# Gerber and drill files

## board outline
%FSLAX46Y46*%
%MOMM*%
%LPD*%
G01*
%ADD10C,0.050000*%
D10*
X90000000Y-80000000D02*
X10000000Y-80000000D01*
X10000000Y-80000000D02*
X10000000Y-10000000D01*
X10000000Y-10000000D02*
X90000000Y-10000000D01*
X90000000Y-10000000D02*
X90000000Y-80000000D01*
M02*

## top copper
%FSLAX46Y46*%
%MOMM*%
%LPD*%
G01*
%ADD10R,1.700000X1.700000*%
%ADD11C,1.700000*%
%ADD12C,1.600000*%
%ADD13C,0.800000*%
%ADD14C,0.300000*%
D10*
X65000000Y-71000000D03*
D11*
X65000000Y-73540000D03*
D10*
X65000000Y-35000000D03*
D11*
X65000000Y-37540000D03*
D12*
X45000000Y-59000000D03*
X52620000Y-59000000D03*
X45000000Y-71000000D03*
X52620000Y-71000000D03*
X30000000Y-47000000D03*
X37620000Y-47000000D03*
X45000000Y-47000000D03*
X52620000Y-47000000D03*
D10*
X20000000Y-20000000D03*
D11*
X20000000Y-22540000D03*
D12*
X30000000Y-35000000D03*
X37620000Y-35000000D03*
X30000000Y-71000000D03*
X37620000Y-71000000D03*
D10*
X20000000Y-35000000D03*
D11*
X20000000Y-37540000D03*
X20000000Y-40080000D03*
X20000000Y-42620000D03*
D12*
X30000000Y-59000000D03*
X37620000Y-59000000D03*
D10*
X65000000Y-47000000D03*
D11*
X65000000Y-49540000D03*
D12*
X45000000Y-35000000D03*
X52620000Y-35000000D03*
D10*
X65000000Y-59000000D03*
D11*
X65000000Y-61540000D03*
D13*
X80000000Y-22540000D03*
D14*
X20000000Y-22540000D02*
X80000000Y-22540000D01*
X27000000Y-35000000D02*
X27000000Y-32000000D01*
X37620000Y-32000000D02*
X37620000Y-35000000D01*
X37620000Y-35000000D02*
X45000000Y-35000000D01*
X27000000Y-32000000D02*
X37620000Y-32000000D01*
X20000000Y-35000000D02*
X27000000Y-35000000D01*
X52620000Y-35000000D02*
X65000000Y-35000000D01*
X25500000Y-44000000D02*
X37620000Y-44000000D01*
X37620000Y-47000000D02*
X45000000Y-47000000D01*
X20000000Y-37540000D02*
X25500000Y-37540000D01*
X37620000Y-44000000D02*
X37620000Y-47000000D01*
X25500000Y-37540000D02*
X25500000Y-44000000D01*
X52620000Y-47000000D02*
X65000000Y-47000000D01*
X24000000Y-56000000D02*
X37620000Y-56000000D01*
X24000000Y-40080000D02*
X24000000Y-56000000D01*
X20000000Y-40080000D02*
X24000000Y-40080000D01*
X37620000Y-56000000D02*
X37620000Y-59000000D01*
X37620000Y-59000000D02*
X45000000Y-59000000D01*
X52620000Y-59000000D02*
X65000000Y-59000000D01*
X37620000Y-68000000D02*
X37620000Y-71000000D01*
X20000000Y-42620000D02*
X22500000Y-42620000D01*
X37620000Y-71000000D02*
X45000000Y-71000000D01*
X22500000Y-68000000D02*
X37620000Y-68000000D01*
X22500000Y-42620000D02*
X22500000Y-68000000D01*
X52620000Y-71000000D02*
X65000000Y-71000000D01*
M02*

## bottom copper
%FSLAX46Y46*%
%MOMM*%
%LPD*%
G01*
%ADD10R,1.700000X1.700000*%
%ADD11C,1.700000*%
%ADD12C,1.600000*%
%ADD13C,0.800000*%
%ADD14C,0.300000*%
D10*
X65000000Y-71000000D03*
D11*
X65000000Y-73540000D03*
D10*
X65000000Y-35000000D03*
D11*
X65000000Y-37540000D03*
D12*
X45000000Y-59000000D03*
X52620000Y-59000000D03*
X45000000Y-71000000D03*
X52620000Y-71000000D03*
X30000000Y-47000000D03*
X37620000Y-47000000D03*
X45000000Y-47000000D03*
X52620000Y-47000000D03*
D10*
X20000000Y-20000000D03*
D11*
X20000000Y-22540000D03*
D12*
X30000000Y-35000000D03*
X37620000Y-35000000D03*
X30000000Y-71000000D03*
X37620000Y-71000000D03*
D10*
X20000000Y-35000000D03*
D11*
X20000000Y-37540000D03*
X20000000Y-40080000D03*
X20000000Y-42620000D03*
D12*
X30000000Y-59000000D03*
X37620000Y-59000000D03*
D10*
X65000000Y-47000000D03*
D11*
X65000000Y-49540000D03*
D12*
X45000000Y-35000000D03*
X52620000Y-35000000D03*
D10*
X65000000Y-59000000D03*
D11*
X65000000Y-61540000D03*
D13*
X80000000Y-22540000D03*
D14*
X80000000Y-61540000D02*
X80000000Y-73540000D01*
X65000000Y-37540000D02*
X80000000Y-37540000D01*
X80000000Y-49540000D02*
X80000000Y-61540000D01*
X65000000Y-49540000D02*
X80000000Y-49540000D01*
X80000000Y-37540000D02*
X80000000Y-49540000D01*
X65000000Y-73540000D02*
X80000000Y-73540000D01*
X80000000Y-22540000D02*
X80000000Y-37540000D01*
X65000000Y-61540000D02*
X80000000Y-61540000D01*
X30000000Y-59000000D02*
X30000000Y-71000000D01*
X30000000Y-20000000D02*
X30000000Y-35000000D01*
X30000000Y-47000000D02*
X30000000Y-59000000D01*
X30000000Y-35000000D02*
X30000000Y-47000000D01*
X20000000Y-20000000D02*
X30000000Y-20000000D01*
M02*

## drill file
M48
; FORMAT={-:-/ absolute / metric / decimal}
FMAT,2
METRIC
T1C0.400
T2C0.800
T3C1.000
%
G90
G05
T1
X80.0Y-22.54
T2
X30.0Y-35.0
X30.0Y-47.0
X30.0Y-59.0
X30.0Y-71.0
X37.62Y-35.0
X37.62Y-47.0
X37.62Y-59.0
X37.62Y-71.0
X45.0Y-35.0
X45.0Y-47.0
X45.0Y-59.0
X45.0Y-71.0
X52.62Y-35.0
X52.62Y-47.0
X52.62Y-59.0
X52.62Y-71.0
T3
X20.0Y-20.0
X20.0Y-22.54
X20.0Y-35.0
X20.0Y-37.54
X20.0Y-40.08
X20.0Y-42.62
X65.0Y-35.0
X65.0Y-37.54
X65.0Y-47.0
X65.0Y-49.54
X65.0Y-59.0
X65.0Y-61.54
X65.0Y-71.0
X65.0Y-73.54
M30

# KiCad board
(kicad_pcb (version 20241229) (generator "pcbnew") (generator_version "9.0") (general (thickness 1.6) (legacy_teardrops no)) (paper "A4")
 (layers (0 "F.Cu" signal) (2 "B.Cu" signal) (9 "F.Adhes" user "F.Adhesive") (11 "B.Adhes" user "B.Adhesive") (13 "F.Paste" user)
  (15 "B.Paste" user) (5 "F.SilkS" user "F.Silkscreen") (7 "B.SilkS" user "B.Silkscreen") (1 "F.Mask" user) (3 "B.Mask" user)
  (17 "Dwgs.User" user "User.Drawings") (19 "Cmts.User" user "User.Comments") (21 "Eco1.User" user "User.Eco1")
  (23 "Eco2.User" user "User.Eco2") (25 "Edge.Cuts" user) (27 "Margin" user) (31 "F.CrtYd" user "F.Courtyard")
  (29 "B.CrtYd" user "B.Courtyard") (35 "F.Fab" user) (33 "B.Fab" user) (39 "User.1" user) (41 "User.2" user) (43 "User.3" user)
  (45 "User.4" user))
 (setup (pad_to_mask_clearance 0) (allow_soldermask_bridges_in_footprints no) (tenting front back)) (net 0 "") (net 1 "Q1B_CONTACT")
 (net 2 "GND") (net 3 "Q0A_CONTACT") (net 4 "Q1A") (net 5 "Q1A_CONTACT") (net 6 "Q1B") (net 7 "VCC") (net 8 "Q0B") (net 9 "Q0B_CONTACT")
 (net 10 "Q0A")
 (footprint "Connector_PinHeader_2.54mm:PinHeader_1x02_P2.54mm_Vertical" (layer "F.Cu") (at 65 71)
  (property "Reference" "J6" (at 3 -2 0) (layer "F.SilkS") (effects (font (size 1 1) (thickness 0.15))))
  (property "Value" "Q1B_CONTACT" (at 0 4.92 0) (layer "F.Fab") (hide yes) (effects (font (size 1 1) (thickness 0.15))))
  (pad "1" thru_hole rect (at 0 0) (size 1.7 1.7) (drill 1) (layers "*.Cu" "*.Mask") (remove_unused_layers no) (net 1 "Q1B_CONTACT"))
  (pad "2" thru_hole circle (at 0 2.54) (size 1.7 1.7) (drill 1) (layers "*.Cu" "*.Mask") (remove_unused_layers no) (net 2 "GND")))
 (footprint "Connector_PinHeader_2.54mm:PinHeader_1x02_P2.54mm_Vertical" (layer "F.Cu") (at 65 35)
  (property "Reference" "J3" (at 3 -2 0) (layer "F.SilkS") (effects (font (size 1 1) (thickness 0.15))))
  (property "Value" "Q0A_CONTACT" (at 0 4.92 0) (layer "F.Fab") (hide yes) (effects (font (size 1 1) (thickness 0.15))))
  (pad "1" thru_hole rect (at 0 0) (size 1.7 1.7) (drill 1) (layers "*.Cu" "*.Mask") (remove_unused_layers no) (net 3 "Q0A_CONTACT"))
  (pad "2" thru_hole circle (at 0 2.54) (size 1.7 1.7) (drill 1) (layers "*.Cu" "*.Mask") (remove_unused_layers no) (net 2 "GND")))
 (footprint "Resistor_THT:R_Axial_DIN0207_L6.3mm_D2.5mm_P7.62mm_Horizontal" (layer "F.Cu") (at 45 59)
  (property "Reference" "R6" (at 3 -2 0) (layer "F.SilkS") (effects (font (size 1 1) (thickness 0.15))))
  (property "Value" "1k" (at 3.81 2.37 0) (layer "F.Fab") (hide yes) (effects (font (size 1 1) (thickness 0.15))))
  (pad "1" thru_hole circle (at 0 0) (size 1.6 1.6) (drill 0.8) (layers "*.Cu" "*.Mask") (remove_unused_layers no) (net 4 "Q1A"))
  (pad "2" thru_hole circle (at 7.62 0) (size 1.6 1.6) (drill 0.8) (layers "*.Cu" "*.Mask") (remove_unused_layers no) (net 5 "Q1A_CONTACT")))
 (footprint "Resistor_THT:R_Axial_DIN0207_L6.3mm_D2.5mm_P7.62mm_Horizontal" (layer "F.Cu") (at 45 71)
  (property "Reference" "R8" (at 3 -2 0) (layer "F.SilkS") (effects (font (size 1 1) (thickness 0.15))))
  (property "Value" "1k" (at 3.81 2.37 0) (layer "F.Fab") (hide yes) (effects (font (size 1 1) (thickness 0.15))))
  (pad "1" thru_hole circle (at 0 0) (size 1.6 1.6) (drill 0.8) (layers "*.Cu" "*.Mask") (remove_unused_layers no) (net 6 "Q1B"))
  (pad "2" thru_hole circle (at 7.62 0) (size 1.6 1.6) (drill 0.8) (layers "*.Cu" "*.Mask") (remove_unused_layers no) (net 1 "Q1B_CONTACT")))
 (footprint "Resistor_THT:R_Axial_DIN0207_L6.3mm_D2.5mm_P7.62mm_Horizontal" (layer "F.Cu") (at 30 47)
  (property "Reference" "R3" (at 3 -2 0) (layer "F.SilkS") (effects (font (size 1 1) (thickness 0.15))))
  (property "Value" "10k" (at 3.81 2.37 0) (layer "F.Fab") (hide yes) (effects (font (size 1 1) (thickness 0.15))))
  (pad "1" thru_hole circle (at 0 0) (size 1.6 1.6) (drill 0.8) (layers "*.Cu" "*.Mask") (remove_unused_layers no) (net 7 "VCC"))
  (pad "2" thru_hole circle (at 7.62 0) (size 1.6 1.6) (drill 0.8) (layers "*.Cu" "*.Mask") (remove_unused_layers no) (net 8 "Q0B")))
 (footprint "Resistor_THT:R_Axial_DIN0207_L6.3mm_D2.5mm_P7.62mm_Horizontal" (layer "F.Cu") (at 45 47)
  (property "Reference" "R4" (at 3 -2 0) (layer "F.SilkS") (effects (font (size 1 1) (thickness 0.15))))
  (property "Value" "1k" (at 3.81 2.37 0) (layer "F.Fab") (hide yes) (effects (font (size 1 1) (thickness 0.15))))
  (pad "1" thru_hole circle (at 0 0) (size 1.6 1.6) (drill 0.8) (layers "*.Cu" "*.Mask") (remove_unused_layers no) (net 8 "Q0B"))
  (pad "2" thru_hole circle (at 7.62 0) (size 1.6 1.6) (drill 0.8) (layers "*.Cu" "*.Mask") (remove_unused_layers no) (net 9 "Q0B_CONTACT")))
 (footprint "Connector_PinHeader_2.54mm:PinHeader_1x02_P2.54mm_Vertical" (layer "F.Cu") (at 20 20)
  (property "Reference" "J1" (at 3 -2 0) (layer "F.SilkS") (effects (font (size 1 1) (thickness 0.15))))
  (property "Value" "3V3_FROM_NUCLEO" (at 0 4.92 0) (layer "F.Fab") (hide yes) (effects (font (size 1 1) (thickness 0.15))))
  (pad "1" thru_hole rect (at 0 0) (size 1.7 1.7) (drill 1) (layers "*.Cu" "*.Mask") (remove_unused_layers no) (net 7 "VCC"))
  (pad "2" thru_hole circle (at 0 2.54) (size 1.7 1.7) (drill 1) (layers "*.Cu" "*.Mask") (remove_unused_layers no) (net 2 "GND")))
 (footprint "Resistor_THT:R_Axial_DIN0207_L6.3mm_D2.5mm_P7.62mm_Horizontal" (layer "F.Cu") (at 30 35)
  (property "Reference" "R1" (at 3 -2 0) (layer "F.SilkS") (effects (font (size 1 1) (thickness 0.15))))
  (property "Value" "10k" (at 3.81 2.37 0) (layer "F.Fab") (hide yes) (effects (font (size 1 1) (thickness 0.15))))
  (pad "1" thru_hole circle (at 0 0) (size 1.6 1.6) (drill 0.8) (layers "*.Cu" "*.Mask") (remove_unused_layers no) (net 7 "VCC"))
  (pad "2" thru_hole circle (at 7.62 0) (size 1.6 1.6) (drill 0.8) (layers "*.Cu" "*.Mask") (remove_unused_layers no) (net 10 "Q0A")))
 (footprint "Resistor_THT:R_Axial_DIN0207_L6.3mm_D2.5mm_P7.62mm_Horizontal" (layer "F.Cu") (at 30 71)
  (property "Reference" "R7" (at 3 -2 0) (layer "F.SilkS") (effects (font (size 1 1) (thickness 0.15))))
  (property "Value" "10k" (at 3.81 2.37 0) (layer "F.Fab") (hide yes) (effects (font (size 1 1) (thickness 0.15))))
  (pad "1" thru_hole circle (at 0 0) (size 1.6 1.6) (drill 0.8) (layers "*.Cu" "*.Mask") (remove_unused_layers no) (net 7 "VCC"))
  (pad "2" thru_hole circle (at 7.62 0) (size 1.6 1.6) (drill 0.8) (layers "*.Cu" "*.Mask") (remove_unused_layers no) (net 6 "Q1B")))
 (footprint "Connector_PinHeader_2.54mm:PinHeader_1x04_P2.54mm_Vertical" (layer "F.Cu") (at 20 35)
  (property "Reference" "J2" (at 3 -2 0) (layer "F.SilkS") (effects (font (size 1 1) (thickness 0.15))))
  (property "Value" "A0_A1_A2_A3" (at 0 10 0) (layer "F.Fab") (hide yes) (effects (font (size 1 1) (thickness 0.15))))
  (pad "1" thru_hole rect (at 0 0) (size 1.7 1.7) (drill 1) (layers "*.Cu" "*.Mask") (remove_unused_layers no) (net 10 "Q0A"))
  (pad "2" thru_hole circle (at 0 2.54) (size 1.7 1.7) (drill 1) (layers "*.Cu" "*.Mask") (remove_unused_layers no) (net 8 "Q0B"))
  (pad "3" thru_hole circle (at 0 5.08) (size 1.7 1.7) (drill 1) (layers "*.Cu" "*.Mask") (remove_unused_layers no) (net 4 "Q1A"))
  (pad "4" thru_hole circle (at 0 7.62) (size 1.7 1.7) (drill 1) (layers "*.Cu" "*.Mask") (remove_unused_layers no) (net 6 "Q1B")))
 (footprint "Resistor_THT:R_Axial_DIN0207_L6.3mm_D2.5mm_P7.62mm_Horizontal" (layer "F.Cu") (at 30 59)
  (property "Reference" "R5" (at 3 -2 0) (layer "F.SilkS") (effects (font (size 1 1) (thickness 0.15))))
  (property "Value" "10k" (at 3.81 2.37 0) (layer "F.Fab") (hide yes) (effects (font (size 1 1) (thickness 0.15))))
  (pad "1" thru_hole circle (at 0 0) (size 1.6 1.6) (drill 0.8) (layers "*.Cu" "*.Mask") (remove_unused_layers no) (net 7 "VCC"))
  (pad "2" thru_hole circle (at 7.62 0) (size 1.6 1.6) (drill 0.8) (layers "*.Cu" "*.Mask") (remove_unused_layers no) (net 4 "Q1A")))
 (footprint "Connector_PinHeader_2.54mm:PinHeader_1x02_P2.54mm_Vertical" (layer "F.Cu") (at 65 47)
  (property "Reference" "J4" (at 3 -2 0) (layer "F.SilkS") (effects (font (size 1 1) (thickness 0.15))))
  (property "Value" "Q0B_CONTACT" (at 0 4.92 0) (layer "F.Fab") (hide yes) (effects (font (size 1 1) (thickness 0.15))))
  (pad "1" thru_hole rect (at 0 0) (size 1.7 1.7) (drill 1) (layers "*.Cu" "*.Mask") (remove_unused_layers no) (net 9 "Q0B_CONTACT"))
  (pad "2" thru_hole circle (at 0 2.54) (size 1.7 1.7) (drill 1) (layers "*.Cu" "*.Mask") (remove_unused_layers no) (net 2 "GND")))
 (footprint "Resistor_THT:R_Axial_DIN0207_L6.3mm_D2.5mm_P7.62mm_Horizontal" (layer "F.Cu") (at 45 35)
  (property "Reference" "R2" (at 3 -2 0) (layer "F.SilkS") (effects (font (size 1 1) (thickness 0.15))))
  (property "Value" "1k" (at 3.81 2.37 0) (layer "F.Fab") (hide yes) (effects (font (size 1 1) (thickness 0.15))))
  (pad "1" thru_hole circle (at 0 0) (size 1.6 1.6) (drill 0.8) (layers "*.Cu" "*.Mask") (remove_unused_layers no) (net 10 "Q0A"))
  (pad "2" thru_hole circle (at 7.62 0) (size 1.6 1.6) (drill 0.8) (layers "*.Cu" "*.Mask") (remove_unused_layers no) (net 3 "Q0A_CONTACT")))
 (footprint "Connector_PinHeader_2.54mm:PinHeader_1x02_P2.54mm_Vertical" (layer "F.Cu") (at 65 59)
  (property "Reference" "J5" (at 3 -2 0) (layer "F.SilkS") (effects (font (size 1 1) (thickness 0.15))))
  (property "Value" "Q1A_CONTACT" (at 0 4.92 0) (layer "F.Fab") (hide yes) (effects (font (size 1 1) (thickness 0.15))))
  (pad "1" thru_hole rect (at 0 0) (size 1.7 1.7) (drill 1) (layers "*.Cu" "*.Mask") (remove_unused_layers no) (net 5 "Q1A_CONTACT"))
  (pad "2" thru_hole circle (at 0 2.54) (size 1.7 1.7) (drill 1) (layers "*.Cu" "*.Mask") (remove_unused_layers no) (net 2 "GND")))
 (gr_line (start 90 80) (end 10 80) (stroke (width 0.05) (type default)) (layer "Edge.Cuts"))
 (gr_line (start 10 80) (end 10 10) (stroke (width 0.05) (type default)) (layer "Edge.Cuts"))
 (gr_line (start 10 10) (end 90 10) (stroke (width 0.05) (type default)) (layer "Edge.Cuts"))
 (gr_line (start 90 10) (end 90 80) (stroke (width 0.05) (type default)) (layer "Edge.Cuts"))
 (segment (start 20 22.54) (end 80 22.54) (width 0.3) (layer "F.Cu") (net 2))
 (via (at 80 22.54) (size 0.8) (drill 0.4) (layers "F.Cu" "B.Cu") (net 2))
 (segment (start 80 61.54) (end 80 73.54) (width 0.3) (layer "B.Cu") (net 2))
 (segment (start 65 37.54) (end 80 37.54) (width 0.3) (layer "B.Cu") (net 2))
 (segment (start 80 49.54) (end 80 61.54) (width 0.3) (layer "B.Cu") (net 2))
 (segment (start 65 49.54) (end 80 49.54) (width 0.3) (layer "B.Cu") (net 2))
 (segment (start 80 37.54) (end 80 49.54) (width 0.3) (layer "B.Cu") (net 2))
 (segment (start 65 73.54) (end 80 73.54) (width 0.3) (layer "B.Cu") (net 2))
 (segment (start 80 22.54) (end 80 37.54) (width 0.3) (layer "B.Cu") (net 2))
 (segment (start 65 61.54) (end 80 61.54) (width 0.3) (layer "B.Cu") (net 2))
 (segment (start 27 35) (end 27 32) (width 0.3) (layer "F.Cu") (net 10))
 (segment (start 37.62 32) (end 37.62 35) (width 0.3) (layer "F.Cu") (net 10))
 (segment (start 37.62 35) (end 45 35) (width 0.3) (layer "F.Cu") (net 10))
 (segment (start 27 32) (end 37.62 32) (width 0.3) (layer "F.Cu") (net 10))
 (segment (start 20 35) (end 27 35) (width 0.3) (layer "F.Cu") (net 10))
 (segment (start 52.62 35) (end 65 35) (width 0.3) (layer "F.Cu") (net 3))
 (segment (start 25.5 44) (end 37.62 44) (width 0.3) (layer "F.Cu") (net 8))
 (segment (start 37.62 47) (end 45 47) (width 0.3) (layer "F.Cu") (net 8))
 (segment (start 20 37.54) (end 25.5 37.54) (width 0.3) (layer "F.Cu") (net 8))
 (segment (start 37.62 44) (end 37.62 47) (width 0.3) (layer "F.Cu") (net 8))
 (segment (start 25.5 37.54) (end 25.5 44) (width 0.3) (layer "F.Cu") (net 8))
 (segment (start 52.62 47) (end 65 47) (width 0.3) (layer "F.Cu") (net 9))
 (segment (start 24 56) (end 37.62 56) (width 0.3) (layer "F.Cu") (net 4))
 (segment (start 24 40.08) (end 24 56) (width 0.3) (layer "F.Cu") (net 4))
 (segment (start 20 40.08) (end 24 40.08) (width 0.3) (layer "F.Cu") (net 4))
 (segment (start 37.62 56) (end 37.62 59) (width 0.3) (layer "F.Cu") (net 4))
 (segment (start 37.62 59) (end 45 59) (width 0.3) (layer "F.Cu") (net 4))
 (segment (start 52.62 59) (end 65 59) (width 0.3) (layer "F.Cu") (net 5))
 (segment (start 37.62 68) (end 37.62 71) (width 0.3) (layer "F.Cu") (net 6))
 (segment (start 20 42.62) (end 22.5 42.62) (width 0.3) (layer "F.Cu") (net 6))
 (segment (start 37.62 71) (end 45 71) (width 0.3) (layer "F.Cu") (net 6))
 (segment (start 22.5 68) (end 37.62 68) (width 0.3) (layer "F.Cu") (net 6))
 (segment (start 22.5 42.62) (end 22.5 68) (width 0.3) (layer "F.Cu") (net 6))
 (segment (start 52.62 71) (end 65 71) (width 0.3) (layer "F.Cu") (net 1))
 (segment (start 30 59) (end 30 71) (width 0.3) (layer "B.Cu") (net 7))
 (segment (start 30 20) (end 30 35) (width 0.3) (layer "B.Cu") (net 7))
 (segment (start 30 47) (end 30 59) (width 0.3) (layer "B.Cu") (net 7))
 (segment (start 30 35) (end 30 47) (width 0.3) (layer "B.Cu") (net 7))
 (segment (start 20 20) (end 30 20) (width 0.3) (layer "B.Cu") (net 7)))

